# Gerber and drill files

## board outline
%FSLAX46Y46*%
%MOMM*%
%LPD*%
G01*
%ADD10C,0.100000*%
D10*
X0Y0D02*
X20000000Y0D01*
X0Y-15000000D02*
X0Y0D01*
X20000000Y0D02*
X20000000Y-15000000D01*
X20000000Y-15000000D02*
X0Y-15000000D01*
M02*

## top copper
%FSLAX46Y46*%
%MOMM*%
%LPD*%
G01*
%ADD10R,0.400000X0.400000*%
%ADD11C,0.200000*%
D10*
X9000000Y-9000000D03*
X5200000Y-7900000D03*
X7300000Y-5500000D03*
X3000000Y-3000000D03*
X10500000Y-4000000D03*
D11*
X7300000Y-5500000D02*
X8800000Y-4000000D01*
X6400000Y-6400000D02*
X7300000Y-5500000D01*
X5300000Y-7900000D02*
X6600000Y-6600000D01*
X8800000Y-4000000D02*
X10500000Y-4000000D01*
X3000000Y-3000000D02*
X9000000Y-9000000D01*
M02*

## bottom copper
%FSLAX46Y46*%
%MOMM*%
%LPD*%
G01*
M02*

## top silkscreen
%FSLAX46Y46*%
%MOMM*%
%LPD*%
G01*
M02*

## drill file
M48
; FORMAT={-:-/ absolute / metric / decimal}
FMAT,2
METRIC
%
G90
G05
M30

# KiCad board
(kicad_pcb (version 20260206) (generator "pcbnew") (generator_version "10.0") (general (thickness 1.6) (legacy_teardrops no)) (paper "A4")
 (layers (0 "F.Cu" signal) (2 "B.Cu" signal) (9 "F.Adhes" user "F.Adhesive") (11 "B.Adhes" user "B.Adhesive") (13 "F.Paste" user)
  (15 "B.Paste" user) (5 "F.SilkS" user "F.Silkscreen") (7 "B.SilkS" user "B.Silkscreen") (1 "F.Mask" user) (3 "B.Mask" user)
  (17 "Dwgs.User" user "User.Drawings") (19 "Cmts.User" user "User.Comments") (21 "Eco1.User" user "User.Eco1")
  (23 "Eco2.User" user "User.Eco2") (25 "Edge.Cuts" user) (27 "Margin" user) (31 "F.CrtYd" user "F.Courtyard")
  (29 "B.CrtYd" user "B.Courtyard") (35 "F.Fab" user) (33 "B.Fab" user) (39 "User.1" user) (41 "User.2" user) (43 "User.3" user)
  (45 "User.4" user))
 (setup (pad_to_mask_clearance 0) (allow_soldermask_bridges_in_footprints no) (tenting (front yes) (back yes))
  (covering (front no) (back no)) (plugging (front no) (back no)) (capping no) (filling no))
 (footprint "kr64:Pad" (layer "F.Cu") (at 9 9)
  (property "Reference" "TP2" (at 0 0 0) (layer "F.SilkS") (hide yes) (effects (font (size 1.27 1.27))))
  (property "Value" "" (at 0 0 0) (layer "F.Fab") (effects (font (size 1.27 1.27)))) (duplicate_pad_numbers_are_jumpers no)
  (pad "1" smd rect (at 0 0) (size 0.4 0.4) (layers "F.Cu" "F.Mask" "F.Paste") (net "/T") (thermal_bridge_angle 45)))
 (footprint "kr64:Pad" (layer "F.Cu") (at 5.2 7.9)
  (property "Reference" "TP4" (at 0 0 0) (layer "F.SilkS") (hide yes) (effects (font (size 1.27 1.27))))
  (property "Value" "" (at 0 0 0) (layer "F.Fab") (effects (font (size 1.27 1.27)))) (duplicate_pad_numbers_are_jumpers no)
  (pad "1" smd rect (at 0 0) (size 0.4 0.4) (layers "F.Cu" "F.Mask" "F.Paste") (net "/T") (thermal_bridge_angle 45)))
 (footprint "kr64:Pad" (layer "F.Cu") (at 7.3 5.5)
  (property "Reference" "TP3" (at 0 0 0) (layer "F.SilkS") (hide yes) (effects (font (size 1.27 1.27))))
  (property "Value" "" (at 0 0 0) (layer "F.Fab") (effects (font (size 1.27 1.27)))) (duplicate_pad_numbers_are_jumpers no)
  (pad "1" smd rect (at 0 0) (size 0.4 0.4) (layers "F.Cu" "F.Mask" "F.Paste") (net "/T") (thermal_bridge_angle 45)))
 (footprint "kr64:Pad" (layer "F.Cu") (at 3 3)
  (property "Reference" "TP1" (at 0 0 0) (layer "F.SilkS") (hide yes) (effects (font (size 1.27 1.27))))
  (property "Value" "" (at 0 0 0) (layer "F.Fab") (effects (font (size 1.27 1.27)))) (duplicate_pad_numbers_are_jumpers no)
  (pad "1" smd rect (at 0 0) (size 0.4 0.4) (layers "F.Cu" "F.Mask" "F.Paste") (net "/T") (thermal_bridge_angle 45)))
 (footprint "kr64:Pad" (layer "F.Cu") (at 10.5 4)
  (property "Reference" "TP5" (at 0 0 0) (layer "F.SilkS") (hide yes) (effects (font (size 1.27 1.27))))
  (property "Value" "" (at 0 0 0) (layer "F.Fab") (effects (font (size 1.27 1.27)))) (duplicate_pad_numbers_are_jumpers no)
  (pad "1" smd rect (at 0 0) (size 0.4 0.4) (layers "F.Cu" "F.Mask" "F.Paste") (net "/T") (thermal_bridge_angle 45)))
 (gr_line (start 0 0) (end 20 0) (stroke (width 0.1) (type default)) (layer "Edge.Cuts"))
 (gr_line (start 0 15) (end 0 0) (stroke (width 0.1) (type default)) (layer "Edge.Cuts"))
 (gr_line (start 20 0) (end 20 15) (stroke (width 0.1) (type default)) (layer "Edge.Cuts"))
 (gr_line (start 20 15) (end 0 15) (stroke (width 0.1) (type default)) (layer "Edge.Cuts"))
 (segment (start 7.3 5.5) (end 8.8 4) (width 0.2) (layer "F.Cu") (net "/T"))
 (segment (start 6.4 6.4) (end 7.3 5.5) (width 0.2) (layer "F.Cu") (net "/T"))
 (segment (start 5.3 7.9) (end 6.6 6.6) (width 0.2) (layer "F.Cu") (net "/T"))
 (segment (start 8.8 4) (end 10.5 4) (width 0.2) (layer "F.Cu") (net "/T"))
 (segment (start 3 3) (end 9 9) (width 0.2) (layer "F.Cu") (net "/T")))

